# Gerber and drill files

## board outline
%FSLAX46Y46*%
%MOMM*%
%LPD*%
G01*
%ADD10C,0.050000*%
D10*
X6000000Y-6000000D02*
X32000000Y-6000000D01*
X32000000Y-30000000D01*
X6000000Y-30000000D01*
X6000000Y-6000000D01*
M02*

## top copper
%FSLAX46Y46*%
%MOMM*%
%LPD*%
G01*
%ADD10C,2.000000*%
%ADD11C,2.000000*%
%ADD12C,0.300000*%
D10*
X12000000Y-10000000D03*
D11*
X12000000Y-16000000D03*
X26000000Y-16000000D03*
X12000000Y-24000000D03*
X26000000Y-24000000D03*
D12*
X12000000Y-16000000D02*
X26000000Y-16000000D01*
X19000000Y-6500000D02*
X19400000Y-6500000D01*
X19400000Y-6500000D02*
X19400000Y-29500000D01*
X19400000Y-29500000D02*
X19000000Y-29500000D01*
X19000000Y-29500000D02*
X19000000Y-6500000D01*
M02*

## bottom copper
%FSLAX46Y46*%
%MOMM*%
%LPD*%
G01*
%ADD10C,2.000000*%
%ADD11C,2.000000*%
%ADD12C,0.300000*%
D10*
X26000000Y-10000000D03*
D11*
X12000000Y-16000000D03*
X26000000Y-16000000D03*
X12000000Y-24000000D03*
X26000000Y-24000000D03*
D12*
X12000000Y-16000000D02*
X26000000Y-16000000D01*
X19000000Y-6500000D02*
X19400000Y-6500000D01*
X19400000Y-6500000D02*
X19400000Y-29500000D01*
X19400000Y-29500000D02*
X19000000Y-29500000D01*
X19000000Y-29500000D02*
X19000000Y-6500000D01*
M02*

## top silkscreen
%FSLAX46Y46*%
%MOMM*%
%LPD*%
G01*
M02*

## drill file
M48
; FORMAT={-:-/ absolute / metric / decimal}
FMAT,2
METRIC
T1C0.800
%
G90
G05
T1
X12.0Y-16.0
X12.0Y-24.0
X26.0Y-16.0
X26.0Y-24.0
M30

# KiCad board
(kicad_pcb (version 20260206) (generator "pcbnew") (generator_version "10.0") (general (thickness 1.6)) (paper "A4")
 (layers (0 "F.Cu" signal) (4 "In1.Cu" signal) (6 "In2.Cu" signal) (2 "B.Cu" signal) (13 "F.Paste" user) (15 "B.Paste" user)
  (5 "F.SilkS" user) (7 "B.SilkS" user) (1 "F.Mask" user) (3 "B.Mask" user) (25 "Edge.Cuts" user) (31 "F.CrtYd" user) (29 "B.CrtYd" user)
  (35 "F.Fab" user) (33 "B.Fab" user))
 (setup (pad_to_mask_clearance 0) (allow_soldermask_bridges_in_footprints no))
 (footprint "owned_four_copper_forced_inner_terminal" (layer "F.Cu") (at 12 10)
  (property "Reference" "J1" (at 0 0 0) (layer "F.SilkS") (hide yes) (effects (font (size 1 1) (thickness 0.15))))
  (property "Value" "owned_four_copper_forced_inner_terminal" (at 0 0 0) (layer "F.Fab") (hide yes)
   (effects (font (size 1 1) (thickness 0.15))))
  (pad "1" smd circle (at 0 0) (size 2 2) (layers "F.Cu" "F.Paste" "F.Mask") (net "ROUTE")))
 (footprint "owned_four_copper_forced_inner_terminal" (layer "B.Cu") (at 26 10)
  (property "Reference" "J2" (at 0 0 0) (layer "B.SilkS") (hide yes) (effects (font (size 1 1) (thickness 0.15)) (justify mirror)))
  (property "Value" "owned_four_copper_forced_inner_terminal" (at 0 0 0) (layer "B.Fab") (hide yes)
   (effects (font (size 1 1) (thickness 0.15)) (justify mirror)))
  (pad "1" smd circle (at 0 0) (size 2 2) (layers "B.Cu" "B.Paste" "B.Mask") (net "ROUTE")))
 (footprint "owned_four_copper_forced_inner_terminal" (layer "F.Cu") (at 12 16)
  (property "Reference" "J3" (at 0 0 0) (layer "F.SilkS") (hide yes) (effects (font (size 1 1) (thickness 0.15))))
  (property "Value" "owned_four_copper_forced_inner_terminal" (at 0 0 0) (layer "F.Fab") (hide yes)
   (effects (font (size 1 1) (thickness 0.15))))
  (pad "1" thru_hole circle (at 0 0) (size 2 2) (drill 0.8) (layers "*.Cu" "*.Mask") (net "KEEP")))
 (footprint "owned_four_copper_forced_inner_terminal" (layer "F.Cu") (at 26 16)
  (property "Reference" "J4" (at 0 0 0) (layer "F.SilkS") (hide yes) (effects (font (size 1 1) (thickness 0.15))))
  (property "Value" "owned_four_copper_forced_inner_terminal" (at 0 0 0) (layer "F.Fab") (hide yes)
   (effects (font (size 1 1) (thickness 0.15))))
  (pad "1" thru_hole circle (at 0 0) (size 2 2) (drill 0.8) (layers "*.Cu" "*.Mask") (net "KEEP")))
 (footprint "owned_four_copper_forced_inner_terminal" (layer "F.Cu") (at 12 24)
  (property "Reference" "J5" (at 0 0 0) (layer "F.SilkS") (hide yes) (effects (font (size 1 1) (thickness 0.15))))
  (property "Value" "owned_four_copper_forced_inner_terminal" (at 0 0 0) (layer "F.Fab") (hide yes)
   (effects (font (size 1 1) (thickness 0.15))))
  (pad "1" thru_hole circle (at 0 0) (size 2 2) (drill 0.8) (layers "*.Cu" "*.Mask") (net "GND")))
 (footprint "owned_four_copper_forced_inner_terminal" (layer "F.Cu") (at 26 24)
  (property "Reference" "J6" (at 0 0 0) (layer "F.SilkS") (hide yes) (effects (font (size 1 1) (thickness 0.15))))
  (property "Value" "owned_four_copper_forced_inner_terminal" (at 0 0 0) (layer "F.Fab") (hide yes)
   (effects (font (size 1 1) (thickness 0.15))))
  (pad "1" thru_hole circle (at 0 0) (size 2 2) (drill 0.8) (layers "*.Cu" "*.Mask") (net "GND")))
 (gr_rect (start 6 6) (end 32 30) (stroke (width 0.05) (type default)) (fill none) (layer "Edge.Cuts"))
 (segment (start 12 16) (end 26 16) (width 0.3) (layer "F.Cu") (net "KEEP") (locked yes))
 (segment (start 12 16) (end 26 16) (width 0.3) (layer "B.Cu") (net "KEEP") (locked yes))
 (segment (start 19 6.5) (end 19.4 6.5) (width 0.3) (layer "F.Cu") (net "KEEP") (locked yes))
 (segment (start 19.4 6.5) (end 19.4 29.5) (width 0.3) (layer "F.Cu") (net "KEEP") (locked yes))
 (segment (start 19.4 29.5) (end 19 29.5) (width 0.3) (layer "F.Cu") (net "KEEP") (locked yes))
 (segment (start 19 29.5) (end 19 6.5) (width 0.3) (layer "F.Cu") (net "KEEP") (locked yes))
 (segment (start 19 6.5) (end 19.4 6.5) (width 0.3) (layer "B.Cu") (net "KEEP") (locked yes))
 (segment (start 19.4 6.5) (end 19.4 29.5) (width 0.3) (layer "B.Cu") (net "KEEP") (locked yes))
 (segment (start 19.4 29.5) (end 19 29.5) (width 0.3) (layer "B.Cu") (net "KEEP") (locked yes))
 (segment (start 19 29.5) (end 19 6.5) (width 0.3) (layer "B.Cu") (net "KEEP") (locked yes)))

